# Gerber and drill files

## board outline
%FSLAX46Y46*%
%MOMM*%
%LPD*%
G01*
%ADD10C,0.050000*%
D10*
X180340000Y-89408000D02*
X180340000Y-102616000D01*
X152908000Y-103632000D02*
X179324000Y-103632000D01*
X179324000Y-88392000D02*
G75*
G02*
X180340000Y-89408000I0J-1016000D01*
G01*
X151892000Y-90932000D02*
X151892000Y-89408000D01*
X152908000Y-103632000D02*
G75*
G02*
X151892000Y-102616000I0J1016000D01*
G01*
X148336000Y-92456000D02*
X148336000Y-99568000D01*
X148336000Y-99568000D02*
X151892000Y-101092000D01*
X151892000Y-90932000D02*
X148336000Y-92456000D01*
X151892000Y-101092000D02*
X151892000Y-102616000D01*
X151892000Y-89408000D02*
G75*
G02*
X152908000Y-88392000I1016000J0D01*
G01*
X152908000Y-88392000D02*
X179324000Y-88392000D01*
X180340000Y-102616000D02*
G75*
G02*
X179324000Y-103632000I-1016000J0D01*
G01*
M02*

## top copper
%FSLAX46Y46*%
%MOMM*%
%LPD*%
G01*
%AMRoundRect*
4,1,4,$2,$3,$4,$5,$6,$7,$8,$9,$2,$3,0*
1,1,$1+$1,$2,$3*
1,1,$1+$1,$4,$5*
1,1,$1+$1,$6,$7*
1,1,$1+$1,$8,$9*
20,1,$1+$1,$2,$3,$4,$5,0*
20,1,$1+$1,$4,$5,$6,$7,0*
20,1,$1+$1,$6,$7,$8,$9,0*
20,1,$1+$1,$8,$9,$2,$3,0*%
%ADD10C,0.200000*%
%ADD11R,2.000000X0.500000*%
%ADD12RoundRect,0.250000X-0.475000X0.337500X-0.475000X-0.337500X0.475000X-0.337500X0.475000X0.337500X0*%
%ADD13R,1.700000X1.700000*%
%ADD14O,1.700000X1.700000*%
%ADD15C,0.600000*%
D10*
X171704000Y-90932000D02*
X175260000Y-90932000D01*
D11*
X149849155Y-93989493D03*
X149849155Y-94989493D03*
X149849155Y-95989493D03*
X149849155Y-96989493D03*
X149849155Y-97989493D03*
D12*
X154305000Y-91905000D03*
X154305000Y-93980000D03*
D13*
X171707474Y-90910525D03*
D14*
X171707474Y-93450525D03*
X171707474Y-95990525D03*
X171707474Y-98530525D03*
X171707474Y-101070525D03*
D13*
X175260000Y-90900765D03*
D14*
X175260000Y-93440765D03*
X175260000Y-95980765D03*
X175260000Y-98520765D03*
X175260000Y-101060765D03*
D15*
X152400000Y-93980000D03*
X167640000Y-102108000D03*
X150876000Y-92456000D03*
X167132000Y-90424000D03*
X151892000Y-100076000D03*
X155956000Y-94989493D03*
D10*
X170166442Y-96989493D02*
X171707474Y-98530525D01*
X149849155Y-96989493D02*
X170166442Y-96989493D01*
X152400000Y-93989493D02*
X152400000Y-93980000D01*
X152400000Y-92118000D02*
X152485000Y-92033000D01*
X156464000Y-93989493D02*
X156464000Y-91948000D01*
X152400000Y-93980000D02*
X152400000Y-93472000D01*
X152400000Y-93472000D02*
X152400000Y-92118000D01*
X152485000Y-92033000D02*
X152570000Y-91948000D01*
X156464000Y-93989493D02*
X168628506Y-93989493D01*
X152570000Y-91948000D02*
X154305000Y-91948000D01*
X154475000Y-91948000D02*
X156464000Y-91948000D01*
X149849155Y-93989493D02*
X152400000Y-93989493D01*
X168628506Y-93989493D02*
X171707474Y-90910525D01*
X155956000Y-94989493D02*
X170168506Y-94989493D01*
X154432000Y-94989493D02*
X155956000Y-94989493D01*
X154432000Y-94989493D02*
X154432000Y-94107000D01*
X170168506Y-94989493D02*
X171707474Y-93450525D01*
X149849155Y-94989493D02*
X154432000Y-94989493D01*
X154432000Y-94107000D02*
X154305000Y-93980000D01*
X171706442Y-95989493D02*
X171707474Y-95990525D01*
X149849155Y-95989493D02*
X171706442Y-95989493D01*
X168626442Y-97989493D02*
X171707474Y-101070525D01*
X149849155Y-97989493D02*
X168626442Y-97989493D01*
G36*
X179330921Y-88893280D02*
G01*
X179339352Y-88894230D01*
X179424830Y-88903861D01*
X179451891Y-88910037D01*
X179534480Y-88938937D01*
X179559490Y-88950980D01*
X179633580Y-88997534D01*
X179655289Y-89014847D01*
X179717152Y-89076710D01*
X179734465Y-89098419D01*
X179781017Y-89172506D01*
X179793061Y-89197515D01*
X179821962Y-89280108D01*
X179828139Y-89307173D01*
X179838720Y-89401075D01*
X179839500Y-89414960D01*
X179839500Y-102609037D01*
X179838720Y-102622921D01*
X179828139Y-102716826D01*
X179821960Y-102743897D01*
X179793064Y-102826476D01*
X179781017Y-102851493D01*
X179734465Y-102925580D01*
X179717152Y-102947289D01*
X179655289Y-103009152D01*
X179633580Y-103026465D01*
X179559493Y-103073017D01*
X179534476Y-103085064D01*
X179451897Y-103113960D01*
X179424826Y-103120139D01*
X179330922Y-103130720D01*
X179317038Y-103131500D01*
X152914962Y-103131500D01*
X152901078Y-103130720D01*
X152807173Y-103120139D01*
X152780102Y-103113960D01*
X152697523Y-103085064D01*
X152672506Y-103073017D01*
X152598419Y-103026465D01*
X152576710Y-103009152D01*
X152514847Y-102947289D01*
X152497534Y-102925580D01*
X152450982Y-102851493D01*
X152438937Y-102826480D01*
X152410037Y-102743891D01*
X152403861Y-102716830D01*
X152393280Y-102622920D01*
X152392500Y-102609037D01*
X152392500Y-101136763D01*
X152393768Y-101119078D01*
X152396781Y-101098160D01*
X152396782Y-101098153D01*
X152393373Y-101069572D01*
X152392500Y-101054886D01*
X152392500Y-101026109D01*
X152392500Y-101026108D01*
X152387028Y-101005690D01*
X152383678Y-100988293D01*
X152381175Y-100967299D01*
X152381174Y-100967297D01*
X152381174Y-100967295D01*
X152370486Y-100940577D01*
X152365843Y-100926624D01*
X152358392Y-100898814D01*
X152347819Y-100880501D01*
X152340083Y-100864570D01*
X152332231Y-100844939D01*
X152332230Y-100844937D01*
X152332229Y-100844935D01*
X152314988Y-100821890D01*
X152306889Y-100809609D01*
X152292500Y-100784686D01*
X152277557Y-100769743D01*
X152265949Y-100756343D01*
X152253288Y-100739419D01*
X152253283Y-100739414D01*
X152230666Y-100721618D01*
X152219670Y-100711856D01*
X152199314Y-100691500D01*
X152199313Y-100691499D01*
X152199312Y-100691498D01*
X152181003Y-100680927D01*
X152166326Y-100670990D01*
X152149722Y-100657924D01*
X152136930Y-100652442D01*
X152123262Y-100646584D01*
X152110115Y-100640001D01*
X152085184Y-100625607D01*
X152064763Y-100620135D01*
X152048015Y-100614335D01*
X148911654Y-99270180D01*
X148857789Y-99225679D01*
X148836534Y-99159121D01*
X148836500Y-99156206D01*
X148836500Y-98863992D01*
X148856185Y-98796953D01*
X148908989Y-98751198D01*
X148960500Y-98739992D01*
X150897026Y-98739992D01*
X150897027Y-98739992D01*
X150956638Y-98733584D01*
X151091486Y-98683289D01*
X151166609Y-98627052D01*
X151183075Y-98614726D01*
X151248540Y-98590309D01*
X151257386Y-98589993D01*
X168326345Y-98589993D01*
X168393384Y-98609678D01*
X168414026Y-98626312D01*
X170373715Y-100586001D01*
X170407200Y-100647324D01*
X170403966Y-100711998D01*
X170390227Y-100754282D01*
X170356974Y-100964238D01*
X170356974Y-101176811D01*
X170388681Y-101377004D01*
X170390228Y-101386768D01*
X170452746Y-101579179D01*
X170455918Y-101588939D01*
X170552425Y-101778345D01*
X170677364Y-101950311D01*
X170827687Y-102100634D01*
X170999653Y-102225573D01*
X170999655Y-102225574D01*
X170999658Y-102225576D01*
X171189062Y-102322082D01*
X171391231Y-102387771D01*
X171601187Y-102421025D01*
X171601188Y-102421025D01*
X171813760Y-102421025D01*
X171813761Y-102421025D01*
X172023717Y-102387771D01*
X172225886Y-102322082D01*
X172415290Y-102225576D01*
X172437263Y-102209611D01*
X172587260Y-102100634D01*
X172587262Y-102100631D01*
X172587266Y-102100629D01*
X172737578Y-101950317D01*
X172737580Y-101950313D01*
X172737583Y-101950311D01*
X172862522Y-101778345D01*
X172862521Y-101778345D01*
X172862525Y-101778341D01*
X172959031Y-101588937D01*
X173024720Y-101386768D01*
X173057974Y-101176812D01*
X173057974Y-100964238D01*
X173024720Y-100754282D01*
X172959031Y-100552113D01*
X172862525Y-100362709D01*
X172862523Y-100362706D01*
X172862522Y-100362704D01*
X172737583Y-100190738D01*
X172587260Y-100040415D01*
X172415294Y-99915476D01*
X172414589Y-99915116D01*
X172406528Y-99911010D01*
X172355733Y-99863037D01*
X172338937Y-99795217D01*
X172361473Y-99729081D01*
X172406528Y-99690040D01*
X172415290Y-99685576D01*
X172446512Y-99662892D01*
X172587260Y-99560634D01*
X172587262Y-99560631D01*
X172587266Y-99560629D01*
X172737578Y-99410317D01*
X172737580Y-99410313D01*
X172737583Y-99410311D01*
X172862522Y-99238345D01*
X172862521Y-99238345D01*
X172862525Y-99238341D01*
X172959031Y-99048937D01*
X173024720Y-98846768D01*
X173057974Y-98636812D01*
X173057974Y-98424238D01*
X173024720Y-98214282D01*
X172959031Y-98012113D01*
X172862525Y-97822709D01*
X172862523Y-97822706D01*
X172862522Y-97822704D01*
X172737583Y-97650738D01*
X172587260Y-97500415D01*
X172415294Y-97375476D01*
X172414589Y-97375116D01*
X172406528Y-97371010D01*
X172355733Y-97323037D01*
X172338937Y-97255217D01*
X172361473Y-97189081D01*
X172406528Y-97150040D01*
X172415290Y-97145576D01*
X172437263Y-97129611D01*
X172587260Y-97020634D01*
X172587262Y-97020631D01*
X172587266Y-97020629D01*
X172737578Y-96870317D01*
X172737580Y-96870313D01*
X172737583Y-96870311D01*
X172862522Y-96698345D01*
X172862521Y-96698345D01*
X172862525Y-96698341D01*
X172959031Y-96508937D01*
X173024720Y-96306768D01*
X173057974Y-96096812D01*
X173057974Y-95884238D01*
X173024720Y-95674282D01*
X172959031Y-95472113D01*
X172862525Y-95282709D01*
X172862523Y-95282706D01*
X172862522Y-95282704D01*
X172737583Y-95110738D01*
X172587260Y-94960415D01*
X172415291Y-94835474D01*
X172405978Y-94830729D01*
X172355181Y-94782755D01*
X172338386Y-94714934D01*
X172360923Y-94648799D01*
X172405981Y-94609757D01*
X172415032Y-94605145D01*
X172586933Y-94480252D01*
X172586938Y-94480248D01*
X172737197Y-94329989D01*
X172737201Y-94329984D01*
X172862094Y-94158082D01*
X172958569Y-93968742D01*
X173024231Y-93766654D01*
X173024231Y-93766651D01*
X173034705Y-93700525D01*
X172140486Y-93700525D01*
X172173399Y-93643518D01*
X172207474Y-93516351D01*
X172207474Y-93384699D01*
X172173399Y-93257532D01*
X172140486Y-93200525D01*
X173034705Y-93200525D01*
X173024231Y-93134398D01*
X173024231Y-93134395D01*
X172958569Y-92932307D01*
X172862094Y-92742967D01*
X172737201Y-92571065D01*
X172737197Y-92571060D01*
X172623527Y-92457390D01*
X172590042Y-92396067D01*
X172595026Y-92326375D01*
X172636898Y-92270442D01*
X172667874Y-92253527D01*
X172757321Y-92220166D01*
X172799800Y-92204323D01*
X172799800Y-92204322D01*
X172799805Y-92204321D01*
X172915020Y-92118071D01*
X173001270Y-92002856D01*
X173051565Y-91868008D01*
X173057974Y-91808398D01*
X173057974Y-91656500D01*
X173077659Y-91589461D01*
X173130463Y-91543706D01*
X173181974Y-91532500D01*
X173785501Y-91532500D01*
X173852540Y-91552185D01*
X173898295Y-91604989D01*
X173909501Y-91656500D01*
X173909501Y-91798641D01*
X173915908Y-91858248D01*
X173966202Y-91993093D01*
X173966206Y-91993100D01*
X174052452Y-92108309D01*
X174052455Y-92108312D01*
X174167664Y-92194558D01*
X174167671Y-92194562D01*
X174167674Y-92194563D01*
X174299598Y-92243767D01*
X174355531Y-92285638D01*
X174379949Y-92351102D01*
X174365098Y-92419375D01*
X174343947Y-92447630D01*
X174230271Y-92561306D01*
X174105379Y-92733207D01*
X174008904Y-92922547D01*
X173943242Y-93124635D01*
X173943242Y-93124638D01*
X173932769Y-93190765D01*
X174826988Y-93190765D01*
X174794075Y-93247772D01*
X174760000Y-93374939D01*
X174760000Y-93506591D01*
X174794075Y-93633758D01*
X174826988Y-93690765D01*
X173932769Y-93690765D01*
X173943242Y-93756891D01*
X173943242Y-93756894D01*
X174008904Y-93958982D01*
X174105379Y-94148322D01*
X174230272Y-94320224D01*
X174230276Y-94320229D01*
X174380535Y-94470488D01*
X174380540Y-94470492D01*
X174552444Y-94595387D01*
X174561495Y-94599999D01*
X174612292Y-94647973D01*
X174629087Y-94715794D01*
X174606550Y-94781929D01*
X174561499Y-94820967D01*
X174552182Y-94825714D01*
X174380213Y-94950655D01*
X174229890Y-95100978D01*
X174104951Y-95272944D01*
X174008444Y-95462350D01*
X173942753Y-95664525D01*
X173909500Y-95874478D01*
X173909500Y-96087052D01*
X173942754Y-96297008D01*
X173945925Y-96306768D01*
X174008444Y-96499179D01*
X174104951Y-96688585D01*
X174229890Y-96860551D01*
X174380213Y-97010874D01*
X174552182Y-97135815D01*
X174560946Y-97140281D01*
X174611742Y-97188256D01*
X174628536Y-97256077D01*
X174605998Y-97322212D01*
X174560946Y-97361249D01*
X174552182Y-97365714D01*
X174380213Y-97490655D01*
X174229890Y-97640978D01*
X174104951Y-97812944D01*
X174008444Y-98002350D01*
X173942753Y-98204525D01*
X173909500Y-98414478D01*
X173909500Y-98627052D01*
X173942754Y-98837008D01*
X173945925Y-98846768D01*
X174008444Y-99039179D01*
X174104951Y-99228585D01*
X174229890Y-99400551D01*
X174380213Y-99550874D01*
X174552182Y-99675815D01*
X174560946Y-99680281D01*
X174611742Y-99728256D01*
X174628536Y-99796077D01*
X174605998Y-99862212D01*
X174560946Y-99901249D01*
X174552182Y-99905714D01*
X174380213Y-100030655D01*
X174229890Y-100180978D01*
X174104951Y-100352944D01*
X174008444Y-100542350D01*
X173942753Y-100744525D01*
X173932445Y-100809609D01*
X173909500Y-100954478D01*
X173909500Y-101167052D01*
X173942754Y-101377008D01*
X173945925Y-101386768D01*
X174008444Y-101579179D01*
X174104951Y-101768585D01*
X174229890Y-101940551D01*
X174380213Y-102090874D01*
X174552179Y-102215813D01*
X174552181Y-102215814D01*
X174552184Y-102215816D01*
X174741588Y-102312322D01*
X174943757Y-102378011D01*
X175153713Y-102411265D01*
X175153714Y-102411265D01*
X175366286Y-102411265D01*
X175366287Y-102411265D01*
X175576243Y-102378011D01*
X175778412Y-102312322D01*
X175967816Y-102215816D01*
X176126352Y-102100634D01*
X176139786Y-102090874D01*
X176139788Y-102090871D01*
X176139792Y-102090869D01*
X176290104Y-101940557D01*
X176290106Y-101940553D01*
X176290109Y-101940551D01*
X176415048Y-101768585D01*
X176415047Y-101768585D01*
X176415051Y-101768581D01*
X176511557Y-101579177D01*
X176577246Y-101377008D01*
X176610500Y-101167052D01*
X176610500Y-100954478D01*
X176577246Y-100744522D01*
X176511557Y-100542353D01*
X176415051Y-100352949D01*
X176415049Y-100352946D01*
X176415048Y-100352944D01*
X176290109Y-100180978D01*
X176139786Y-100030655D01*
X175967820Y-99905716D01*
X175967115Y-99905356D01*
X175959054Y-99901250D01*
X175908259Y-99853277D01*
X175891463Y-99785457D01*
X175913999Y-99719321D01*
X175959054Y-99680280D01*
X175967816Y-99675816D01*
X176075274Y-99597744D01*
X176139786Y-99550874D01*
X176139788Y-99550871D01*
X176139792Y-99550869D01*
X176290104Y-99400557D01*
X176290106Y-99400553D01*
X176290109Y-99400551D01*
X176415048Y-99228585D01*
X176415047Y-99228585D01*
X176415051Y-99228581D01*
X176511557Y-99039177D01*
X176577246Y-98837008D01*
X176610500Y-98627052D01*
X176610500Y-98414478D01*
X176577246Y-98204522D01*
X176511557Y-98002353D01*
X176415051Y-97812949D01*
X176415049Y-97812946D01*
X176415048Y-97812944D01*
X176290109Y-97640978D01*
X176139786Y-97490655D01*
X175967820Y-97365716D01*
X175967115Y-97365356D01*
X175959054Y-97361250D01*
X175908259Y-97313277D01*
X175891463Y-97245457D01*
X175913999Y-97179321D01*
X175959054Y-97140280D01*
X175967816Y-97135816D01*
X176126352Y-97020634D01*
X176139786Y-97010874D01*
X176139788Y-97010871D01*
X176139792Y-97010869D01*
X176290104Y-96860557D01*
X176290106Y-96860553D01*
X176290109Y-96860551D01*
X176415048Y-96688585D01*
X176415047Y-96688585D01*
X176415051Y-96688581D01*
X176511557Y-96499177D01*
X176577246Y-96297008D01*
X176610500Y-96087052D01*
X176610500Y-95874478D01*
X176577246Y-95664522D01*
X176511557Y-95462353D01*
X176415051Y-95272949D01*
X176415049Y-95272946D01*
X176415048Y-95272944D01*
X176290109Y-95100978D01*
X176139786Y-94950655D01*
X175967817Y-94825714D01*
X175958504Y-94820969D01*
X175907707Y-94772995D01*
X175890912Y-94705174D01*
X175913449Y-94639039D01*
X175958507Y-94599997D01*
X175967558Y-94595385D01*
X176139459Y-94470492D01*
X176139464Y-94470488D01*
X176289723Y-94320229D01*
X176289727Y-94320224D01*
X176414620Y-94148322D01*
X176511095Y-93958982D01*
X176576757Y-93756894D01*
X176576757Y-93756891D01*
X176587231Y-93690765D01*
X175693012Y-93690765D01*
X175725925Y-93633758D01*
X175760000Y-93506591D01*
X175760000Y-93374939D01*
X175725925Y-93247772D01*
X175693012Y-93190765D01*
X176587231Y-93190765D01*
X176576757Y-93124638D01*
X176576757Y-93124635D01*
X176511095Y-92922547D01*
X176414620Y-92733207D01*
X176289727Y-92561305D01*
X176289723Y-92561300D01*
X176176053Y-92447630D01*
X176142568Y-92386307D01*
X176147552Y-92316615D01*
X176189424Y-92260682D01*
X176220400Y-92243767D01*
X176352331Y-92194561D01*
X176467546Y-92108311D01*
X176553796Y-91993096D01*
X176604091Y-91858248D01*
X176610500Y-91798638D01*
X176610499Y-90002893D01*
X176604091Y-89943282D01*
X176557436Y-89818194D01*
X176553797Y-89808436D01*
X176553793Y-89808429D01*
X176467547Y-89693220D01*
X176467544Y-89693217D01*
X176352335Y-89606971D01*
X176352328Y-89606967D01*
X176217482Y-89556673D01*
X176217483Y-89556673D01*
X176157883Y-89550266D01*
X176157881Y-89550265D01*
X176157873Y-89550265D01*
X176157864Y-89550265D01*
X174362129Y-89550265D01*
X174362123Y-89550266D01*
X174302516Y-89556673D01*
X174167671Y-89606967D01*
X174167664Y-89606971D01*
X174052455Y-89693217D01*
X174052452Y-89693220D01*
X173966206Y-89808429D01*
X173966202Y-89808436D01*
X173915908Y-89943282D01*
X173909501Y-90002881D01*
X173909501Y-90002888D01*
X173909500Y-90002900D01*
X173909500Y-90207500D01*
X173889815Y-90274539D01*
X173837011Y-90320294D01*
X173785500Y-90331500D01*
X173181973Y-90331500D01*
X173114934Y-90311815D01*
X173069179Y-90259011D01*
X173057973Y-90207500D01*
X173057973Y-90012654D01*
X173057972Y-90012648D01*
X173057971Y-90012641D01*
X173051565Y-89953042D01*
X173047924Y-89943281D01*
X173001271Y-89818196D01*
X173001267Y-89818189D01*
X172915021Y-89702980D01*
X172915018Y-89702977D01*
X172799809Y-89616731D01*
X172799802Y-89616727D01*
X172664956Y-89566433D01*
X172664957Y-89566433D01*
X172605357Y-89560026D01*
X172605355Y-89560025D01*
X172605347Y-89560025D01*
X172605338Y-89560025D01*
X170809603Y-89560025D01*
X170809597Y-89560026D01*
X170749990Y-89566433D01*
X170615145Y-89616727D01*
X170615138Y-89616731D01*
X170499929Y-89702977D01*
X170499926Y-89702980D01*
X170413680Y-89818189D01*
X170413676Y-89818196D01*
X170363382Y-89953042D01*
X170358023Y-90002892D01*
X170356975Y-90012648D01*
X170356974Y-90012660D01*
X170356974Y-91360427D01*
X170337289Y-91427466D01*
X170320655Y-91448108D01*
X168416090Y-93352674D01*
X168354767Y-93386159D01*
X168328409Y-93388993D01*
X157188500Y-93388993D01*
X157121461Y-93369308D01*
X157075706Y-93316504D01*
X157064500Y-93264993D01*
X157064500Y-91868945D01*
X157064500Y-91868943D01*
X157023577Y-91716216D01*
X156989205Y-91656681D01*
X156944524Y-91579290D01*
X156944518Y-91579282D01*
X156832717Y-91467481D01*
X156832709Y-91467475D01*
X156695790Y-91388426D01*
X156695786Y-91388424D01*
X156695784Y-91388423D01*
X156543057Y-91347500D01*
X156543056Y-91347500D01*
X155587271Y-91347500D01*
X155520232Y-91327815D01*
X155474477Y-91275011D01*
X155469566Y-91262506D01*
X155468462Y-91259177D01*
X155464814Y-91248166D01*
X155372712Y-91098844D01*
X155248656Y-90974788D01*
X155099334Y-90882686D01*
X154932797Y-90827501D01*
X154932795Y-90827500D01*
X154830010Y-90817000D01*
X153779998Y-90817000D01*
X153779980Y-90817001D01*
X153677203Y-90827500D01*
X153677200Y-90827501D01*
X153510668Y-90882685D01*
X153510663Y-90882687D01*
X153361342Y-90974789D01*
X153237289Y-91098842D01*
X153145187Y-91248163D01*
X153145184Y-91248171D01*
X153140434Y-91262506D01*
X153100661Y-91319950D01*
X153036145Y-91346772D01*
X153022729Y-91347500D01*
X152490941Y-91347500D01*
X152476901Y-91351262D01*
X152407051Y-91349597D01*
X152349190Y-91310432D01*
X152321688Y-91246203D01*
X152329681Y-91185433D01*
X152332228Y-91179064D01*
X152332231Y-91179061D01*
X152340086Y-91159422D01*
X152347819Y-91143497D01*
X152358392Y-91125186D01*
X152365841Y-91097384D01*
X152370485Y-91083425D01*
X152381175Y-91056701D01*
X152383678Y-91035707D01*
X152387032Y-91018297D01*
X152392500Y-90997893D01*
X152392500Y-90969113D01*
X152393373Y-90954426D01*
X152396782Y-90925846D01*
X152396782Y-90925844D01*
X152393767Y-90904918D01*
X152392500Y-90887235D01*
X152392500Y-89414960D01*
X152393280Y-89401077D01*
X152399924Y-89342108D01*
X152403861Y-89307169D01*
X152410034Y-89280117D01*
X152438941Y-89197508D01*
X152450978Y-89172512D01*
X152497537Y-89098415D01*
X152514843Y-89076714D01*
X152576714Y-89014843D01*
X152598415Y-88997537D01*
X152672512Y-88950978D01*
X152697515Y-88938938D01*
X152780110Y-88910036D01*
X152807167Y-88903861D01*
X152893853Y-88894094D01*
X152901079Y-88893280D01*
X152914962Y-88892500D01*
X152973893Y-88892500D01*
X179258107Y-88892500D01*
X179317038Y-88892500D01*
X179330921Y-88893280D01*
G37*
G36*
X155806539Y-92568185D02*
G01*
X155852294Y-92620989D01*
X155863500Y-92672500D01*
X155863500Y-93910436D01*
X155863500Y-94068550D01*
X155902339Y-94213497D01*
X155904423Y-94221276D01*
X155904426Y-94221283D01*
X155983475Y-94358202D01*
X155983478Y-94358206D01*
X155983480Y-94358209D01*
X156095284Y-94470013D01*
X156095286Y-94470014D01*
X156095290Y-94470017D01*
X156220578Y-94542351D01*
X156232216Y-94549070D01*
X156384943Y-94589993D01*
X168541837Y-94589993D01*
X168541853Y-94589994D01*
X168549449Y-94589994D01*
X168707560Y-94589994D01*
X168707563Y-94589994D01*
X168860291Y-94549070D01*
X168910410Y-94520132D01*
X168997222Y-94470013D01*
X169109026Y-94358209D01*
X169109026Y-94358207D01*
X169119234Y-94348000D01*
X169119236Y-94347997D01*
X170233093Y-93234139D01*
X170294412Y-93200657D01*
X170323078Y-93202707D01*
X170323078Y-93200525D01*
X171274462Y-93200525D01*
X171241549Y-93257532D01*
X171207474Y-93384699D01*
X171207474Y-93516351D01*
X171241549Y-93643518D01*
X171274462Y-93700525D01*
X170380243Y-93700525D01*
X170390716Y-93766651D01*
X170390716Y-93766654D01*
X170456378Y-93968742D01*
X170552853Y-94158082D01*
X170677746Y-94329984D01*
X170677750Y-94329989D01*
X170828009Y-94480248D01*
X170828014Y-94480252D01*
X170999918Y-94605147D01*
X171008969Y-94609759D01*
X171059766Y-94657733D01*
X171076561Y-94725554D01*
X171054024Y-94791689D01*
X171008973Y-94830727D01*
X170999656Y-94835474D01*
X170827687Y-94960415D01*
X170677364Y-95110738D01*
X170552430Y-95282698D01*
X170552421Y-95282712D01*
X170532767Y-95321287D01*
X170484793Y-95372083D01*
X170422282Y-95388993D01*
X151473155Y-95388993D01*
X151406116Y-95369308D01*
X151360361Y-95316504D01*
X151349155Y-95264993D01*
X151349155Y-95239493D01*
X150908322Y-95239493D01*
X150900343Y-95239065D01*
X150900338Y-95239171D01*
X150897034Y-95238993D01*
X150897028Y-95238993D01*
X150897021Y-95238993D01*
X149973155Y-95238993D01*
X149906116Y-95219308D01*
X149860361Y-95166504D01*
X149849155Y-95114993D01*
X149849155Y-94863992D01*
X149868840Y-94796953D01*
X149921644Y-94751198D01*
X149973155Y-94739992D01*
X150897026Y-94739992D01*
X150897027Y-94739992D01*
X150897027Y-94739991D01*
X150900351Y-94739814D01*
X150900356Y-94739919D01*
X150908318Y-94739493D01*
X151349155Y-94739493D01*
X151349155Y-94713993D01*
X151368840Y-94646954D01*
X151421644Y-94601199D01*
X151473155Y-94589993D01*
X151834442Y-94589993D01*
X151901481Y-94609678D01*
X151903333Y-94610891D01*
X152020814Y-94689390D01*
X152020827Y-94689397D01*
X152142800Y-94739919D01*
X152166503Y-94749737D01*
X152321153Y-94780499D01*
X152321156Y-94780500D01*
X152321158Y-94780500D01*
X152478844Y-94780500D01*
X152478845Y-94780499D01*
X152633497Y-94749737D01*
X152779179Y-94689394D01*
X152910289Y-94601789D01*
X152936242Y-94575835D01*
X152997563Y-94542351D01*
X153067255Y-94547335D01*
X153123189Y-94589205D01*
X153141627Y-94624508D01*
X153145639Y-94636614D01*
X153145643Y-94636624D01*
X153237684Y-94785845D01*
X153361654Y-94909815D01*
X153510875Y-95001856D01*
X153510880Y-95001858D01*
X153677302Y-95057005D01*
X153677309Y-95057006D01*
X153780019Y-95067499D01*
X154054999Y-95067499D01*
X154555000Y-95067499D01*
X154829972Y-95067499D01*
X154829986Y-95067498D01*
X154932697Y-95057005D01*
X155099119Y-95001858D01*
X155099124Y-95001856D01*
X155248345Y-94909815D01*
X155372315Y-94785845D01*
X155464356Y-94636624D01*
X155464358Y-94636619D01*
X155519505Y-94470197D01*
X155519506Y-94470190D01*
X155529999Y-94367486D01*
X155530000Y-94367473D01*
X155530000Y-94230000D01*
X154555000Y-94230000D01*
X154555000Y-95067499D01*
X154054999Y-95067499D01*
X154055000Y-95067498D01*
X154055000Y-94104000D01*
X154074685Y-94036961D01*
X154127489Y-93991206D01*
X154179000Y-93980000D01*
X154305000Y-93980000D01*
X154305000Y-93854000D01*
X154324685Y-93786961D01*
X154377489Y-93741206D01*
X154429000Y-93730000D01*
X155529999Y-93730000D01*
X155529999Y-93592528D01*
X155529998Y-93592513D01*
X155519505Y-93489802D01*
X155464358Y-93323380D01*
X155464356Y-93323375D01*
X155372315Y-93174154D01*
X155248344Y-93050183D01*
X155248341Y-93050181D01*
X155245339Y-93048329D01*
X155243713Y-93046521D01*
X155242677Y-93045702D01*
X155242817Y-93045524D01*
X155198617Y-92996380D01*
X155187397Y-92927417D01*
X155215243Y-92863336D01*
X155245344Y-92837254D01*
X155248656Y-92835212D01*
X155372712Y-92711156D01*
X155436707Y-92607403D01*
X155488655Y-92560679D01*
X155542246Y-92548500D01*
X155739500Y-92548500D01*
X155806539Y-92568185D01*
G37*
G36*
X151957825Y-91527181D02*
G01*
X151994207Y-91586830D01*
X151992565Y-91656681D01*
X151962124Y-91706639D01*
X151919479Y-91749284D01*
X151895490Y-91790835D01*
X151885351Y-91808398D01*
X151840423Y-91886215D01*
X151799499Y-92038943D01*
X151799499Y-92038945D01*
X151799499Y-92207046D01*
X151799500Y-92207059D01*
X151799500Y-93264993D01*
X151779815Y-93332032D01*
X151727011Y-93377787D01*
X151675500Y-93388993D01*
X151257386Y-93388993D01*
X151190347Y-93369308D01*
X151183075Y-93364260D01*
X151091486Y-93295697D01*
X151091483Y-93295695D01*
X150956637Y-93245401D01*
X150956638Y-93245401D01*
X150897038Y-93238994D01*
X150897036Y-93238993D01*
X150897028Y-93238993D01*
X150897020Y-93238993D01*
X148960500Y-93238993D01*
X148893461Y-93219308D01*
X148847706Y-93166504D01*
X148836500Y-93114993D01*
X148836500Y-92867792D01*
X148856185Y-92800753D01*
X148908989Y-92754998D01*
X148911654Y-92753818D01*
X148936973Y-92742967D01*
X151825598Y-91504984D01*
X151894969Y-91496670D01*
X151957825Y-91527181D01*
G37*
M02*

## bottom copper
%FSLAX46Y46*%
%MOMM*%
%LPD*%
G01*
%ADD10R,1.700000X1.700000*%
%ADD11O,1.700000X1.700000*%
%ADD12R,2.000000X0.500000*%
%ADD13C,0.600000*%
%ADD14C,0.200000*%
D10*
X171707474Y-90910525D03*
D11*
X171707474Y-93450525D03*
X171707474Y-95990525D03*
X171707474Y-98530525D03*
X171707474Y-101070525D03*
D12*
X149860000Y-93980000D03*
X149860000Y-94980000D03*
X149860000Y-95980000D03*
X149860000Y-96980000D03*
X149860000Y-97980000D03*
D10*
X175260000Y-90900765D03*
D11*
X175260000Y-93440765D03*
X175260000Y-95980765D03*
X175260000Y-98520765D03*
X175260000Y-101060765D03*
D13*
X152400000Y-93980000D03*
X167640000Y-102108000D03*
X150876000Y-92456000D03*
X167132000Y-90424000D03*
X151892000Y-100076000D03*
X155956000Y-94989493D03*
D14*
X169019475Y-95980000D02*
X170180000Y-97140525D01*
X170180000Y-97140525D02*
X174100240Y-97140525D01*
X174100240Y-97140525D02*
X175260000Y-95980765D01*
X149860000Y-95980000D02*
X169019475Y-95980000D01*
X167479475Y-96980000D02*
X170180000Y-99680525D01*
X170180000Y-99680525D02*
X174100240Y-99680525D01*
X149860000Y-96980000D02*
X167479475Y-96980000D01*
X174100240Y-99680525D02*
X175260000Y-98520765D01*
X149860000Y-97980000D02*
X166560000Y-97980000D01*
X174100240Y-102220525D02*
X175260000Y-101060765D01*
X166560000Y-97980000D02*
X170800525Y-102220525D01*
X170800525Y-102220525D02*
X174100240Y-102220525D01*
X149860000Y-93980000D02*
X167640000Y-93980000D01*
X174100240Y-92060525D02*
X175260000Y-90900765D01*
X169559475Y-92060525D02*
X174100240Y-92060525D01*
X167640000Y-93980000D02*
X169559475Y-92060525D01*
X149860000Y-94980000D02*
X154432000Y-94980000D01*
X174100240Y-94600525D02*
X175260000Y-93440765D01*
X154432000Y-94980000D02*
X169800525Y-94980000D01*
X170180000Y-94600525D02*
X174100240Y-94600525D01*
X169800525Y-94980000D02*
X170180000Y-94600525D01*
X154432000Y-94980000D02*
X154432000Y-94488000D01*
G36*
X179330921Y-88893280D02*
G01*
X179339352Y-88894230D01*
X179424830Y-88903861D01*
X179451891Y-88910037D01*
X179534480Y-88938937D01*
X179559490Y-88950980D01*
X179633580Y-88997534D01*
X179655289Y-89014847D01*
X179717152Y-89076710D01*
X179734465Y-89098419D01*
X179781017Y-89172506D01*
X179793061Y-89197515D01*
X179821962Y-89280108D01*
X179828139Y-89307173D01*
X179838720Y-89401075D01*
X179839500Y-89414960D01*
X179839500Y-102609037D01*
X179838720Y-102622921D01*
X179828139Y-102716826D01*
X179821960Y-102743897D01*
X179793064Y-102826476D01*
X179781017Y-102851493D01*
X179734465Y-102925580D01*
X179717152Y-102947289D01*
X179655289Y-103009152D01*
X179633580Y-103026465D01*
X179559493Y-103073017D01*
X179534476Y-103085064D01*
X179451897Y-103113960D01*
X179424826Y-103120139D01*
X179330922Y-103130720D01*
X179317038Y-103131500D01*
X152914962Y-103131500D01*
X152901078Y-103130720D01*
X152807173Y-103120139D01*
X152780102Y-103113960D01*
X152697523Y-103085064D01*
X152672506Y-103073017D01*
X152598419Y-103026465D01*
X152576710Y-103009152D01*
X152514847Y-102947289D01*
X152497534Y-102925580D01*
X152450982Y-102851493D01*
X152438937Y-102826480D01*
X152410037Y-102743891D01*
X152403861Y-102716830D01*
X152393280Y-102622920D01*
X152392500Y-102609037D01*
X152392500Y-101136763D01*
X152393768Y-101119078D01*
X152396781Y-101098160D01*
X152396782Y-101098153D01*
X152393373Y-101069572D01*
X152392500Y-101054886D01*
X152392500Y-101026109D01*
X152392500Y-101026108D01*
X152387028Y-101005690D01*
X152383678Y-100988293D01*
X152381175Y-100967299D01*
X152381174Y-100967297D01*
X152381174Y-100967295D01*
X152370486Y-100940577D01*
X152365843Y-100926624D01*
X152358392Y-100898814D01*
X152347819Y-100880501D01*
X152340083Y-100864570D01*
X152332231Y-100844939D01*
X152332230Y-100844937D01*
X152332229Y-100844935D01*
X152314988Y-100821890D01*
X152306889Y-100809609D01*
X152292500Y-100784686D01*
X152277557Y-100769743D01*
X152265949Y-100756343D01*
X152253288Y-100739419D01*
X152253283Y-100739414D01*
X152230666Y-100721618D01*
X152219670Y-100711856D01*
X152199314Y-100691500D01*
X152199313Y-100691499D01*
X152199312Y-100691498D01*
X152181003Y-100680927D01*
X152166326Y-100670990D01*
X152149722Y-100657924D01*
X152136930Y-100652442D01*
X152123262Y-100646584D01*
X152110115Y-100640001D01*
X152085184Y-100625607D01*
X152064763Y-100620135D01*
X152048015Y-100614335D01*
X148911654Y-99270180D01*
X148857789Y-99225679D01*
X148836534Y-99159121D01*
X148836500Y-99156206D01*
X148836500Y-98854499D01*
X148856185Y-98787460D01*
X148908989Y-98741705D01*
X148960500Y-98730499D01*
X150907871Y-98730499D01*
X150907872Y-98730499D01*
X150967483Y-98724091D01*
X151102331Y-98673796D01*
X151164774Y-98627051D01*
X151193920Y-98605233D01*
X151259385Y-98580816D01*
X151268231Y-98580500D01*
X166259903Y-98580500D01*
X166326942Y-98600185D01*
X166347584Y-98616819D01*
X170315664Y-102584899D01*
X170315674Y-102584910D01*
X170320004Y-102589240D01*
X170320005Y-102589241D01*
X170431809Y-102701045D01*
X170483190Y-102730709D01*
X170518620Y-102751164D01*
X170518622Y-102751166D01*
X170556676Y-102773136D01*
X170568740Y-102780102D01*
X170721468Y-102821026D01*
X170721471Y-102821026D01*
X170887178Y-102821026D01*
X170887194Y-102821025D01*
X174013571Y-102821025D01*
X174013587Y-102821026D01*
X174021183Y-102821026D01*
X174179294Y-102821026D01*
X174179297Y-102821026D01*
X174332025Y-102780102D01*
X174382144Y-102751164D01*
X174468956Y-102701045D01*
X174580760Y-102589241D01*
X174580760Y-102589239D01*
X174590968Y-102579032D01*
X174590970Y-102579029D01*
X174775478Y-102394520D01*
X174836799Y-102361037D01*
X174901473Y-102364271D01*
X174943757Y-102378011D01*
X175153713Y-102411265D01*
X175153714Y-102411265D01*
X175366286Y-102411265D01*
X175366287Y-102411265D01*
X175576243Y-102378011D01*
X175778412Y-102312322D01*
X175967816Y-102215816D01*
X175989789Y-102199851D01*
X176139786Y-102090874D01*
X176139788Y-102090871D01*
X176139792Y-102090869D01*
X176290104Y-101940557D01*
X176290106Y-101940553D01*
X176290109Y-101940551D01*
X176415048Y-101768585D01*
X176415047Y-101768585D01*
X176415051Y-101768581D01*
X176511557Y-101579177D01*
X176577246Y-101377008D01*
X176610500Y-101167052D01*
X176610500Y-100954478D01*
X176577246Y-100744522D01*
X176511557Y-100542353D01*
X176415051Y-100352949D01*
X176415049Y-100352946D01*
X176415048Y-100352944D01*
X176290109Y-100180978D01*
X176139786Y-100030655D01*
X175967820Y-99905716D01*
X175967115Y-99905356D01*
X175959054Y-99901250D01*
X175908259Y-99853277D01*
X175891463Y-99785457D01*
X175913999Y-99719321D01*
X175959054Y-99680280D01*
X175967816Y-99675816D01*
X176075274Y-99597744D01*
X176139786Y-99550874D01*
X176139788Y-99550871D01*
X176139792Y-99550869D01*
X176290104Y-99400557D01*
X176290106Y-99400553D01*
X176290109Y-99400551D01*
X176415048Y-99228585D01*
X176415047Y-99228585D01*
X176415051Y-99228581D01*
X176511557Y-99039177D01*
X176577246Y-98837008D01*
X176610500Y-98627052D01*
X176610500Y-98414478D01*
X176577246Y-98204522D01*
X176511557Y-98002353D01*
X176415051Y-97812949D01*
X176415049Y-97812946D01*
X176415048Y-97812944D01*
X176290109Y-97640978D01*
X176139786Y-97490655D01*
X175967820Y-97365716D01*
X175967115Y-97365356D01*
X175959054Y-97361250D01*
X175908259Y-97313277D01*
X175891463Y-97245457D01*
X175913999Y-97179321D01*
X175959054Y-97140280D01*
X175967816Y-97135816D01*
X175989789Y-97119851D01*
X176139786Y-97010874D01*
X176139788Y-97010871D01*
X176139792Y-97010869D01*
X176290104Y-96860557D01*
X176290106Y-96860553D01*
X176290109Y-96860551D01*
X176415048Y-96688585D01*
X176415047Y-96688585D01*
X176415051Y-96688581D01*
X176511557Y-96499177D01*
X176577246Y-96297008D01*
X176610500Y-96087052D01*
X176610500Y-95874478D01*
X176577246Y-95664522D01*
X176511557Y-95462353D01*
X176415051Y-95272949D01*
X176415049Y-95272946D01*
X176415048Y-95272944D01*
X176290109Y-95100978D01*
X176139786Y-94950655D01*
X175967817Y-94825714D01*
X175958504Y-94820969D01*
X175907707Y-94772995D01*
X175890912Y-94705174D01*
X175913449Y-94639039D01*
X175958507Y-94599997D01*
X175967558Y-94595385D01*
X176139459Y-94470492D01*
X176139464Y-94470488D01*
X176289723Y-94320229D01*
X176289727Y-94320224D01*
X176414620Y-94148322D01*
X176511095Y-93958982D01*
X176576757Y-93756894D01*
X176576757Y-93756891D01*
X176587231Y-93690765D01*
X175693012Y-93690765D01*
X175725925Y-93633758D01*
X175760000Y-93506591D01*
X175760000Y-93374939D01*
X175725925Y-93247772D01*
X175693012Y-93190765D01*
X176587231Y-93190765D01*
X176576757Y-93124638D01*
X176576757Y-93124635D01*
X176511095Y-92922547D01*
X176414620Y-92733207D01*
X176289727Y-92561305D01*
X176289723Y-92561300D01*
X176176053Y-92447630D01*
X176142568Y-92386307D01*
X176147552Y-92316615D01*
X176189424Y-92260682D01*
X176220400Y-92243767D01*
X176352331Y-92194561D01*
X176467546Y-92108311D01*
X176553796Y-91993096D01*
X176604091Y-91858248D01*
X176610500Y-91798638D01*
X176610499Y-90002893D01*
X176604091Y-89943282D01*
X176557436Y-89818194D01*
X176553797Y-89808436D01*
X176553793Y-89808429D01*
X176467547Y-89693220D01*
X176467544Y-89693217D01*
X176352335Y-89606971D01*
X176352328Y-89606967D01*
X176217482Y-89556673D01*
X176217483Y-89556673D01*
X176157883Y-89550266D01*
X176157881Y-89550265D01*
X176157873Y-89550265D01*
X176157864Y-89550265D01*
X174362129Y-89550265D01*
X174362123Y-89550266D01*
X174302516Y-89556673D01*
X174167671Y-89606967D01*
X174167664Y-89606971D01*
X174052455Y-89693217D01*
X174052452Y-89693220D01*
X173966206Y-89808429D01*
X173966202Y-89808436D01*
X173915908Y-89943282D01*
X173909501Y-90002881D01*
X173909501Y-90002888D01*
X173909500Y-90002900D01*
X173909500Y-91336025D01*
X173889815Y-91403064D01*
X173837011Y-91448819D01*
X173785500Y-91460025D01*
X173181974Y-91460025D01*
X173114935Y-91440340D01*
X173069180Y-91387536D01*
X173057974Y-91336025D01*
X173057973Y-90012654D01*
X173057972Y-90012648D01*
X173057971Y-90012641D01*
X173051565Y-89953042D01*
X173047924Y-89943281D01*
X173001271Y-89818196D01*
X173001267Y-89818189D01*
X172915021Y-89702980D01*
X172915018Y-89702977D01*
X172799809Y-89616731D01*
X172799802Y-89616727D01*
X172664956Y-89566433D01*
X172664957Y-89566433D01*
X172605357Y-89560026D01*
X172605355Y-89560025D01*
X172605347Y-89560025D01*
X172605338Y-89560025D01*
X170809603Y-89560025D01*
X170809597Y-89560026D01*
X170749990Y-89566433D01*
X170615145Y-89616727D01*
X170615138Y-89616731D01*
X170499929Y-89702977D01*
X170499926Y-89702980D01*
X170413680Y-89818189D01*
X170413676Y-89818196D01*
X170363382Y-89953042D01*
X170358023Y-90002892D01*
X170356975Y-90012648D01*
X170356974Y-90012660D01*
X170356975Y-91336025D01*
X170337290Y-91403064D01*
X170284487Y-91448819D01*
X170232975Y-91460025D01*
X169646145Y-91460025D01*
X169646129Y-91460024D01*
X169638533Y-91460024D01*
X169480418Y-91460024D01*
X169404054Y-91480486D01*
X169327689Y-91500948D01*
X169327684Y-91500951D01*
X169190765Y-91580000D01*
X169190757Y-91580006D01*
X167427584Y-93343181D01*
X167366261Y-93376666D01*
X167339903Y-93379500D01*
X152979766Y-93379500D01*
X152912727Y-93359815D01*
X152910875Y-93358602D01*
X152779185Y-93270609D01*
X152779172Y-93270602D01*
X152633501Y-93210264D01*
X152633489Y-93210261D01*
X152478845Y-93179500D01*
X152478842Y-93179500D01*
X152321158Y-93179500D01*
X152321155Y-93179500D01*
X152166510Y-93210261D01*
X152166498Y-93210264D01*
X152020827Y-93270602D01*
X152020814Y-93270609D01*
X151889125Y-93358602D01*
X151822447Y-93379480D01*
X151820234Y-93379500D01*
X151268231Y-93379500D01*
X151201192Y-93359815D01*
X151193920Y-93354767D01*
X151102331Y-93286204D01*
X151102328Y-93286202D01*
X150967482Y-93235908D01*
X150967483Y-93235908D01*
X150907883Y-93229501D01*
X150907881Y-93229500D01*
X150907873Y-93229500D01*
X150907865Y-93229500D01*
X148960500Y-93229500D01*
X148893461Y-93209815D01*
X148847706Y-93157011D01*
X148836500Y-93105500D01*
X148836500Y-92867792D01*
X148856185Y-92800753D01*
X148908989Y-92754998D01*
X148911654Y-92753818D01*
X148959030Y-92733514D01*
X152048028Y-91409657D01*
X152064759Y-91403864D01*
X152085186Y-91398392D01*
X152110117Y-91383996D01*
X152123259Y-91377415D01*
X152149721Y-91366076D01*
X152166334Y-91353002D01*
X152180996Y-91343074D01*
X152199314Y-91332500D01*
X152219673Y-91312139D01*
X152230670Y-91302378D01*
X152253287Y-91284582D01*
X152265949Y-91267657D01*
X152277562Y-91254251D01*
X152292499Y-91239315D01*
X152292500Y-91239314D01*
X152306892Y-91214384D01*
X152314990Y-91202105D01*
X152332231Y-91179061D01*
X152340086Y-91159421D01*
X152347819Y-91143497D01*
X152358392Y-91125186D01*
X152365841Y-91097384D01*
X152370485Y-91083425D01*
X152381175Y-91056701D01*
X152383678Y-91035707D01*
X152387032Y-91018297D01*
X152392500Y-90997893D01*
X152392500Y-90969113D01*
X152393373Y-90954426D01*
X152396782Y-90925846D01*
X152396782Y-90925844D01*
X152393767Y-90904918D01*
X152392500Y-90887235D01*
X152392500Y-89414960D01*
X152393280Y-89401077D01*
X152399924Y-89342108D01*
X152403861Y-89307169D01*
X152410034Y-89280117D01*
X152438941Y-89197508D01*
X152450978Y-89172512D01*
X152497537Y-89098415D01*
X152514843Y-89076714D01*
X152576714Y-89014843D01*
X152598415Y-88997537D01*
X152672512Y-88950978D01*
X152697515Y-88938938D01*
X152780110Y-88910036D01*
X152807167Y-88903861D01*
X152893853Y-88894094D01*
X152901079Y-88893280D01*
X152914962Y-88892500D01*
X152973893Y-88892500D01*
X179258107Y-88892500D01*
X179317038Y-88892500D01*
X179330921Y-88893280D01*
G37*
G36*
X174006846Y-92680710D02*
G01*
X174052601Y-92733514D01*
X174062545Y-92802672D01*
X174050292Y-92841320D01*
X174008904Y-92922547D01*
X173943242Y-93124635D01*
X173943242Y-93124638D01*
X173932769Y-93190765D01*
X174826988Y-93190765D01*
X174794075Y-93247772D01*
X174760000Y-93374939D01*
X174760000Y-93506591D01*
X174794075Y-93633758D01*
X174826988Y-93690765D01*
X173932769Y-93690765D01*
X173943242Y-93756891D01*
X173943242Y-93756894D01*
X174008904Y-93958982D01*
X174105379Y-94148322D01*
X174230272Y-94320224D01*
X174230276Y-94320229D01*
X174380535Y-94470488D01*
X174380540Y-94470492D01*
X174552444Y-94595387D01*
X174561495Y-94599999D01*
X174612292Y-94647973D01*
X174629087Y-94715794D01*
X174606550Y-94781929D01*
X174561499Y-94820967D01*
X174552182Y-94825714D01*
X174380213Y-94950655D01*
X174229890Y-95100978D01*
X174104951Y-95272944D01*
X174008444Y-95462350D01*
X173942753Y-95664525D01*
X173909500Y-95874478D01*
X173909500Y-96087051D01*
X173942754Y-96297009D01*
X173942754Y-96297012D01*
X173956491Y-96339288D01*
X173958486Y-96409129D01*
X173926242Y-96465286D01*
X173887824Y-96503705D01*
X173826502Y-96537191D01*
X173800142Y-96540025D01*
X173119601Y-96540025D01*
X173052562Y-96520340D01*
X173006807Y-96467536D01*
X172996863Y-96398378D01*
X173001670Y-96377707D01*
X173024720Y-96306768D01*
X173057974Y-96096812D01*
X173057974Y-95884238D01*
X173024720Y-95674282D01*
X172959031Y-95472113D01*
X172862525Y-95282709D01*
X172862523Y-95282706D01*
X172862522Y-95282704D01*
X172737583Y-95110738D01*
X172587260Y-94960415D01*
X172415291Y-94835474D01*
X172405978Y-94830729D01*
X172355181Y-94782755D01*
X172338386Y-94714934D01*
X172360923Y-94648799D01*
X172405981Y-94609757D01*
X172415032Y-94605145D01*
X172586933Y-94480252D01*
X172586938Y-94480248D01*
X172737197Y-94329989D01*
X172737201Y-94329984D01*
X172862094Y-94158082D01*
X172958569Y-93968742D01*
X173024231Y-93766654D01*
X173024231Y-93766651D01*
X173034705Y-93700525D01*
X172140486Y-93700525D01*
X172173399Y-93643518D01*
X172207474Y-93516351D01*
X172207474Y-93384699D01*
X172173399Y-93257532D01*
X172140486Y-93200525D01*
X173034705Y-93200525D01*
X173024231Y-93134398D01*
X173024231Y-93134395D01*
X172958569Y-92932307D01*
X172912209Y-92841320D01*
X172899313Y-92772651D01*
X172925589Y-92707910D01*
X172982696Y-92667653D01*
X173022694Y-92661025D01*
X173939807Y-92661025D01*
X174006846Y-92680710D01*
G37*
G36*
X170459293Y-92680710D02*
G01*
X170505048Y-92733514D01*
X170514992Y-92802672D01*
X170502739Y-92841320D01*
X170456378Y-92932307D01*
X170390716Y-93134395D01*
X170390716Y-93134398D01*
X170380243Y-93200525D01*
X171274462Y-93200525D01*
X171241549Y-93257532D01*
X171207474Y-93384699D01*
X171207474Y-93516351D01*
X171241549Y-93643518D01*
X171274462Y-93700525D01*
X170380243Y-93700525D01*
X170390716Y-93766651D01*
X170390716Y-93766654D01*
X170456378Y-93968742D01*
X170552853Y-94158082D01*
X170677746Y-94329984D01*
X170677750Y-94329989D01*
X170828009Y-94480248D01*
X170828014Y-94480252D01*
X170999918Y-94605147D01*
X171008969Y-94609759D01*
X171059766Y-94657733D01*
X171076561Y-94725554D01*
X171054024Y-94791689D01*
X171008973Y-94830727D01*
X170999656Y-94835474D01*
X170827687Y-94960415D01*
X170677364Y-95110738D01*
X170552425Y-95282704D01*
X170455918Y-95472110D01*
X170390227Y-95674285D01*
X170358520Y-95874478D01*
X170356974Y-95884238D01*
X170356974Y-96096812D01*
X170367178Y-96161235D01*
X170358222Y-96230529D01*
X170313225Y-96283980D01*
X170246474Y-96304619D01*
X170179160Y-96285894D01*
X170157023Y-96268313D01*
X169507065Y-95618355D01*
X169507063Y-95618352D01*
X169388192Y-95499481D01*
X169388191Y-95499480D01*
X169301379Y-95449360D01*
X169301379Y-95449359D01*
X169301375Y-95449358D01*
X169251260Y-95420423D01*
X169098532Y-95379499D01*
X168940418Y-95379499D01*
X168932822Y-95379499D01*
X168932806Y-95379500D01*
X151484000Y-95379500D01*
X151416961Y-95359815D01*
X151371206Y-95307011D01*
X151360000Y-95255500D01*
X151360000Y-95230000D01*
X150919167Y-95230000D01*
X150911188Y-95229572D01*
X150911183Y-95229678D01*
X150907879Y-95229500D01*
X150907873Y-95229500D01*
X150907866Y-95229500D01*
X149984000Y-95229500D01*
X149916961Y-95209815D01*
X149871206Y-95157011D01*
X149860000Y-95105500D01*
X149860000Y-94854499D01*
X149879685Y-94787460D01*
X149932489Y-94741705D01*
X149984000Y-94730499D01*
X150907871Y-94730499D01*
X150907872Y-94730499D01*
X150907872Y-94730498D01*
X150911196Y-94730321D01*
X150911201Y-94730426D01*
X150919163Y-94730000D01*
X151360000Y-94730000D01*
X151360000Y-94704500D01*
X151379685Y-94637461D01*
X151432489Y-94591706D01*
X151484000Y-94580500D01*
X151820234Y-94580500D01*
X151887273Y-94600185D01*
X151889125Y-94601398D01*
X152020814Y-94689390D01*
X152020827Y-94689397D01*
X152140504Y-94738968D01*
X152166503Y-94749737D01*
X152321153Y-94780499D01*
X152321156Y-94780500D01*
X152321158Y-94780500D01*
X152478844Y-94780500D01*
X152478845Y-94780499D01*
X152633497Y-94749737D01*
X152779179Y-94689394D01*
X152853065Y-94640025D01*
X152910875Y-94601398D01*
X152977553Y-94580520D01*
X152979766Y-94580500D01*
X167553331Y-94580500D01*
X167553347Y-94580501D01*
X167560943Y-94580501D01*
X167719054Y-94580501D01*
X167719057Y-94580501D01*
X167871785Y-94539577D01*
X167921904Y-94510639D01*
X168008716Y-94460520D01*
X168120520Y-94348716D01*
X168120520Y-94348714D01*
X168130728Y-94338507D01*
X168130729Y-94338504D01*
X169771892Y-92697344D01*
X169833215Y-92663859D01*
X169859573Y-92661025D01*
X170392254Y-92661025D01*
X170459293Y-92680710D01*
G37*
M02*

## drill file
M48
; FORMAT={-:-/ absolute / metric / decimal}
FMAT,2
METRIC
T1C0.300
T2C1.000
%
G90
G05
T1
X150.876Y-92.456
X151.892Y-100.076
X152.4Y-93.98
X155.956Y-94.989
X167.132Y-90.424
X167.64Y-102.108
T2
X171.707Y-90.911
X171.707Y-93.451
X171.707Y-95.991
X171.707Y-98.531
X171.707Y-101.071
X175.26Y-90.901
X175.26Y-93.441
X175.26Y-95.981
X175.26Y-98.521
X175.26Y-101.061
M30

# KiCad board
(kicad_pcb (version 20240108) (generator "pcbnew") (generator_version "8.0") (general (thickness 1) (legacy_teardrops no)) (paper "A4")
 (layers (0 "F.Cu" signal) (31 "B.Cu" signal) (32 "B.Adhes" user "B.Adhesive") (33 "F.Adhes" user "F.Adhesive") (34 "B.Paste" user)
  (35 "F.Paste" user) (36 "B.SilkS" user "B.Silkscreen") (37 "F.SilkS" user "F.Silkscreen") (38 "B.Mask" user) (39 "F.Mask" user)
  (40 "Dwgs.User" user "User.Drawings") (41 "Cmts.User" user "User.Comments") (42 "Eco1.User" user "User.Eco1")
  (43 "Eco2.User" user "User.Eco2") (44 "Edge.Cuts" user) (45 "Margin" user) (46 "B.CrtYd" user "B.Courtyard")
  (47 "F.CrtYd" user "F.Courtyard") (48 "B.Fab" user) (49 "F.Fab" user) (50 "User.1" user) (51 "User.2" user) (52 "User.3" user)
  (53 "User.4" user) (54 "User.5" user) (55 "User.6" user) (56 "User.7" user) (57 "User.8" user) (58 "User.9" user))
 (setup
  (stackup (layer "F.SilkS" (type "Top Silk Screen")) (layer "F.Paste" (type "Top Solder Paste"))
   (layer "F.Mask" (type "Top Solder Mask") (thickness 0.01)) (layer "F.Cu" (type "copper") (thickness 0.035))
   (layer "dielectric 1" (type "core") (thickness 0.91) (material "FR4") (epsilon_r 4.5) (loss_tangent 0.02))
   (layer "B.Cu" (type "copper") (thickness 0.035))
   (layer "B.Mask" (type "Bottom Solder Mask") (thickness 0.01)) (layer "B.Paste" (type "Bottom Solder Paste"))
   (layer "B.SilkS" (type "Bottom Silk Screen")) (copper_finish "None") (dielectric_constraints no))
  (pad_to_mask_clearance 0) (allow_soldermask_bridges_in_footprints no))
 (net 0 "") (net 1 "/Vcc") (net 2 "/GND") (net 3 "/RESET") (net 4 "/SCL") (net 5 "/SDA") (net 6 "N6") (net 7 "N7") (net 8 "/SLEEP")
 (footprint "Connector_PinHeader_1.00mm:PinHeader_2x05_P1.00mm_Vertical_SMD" (layer "F.Cu") (at 149.874555 95.941493)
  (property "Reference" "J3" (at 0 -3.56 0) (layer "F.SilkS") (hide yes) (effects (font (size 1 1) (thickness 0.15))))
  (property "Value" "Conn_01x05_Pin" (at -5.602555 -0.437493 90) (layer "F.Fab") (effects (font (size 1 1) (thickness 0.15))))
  (pad "1" smd rect (at -0.0254 -1.952) (size 2 0.5) (layers "F.Cu" "F.Paste" "F.Mask") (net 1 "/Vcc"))
  (pad "2" smd rect (at -0.0254 -0.952) (size 2 0.5) (layers "F.Cu" "F.Paste" "F.Mask") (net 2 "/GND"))
  (pad "3" smd rect (at -0.0254 0.048) (size 2 0.5) (layers "F.Cu" "F.Paste" "F.Mask") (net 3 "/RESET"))
  (pad "4" smd rect (at -0.0254 1.048) (size 2 0.5) (layers "F.Cu" "F.Paste" "F.Mask") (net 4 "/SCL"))
  (pad "5" smd rect (at -0.0254 2.048) (size 2 0.5) (layers "F.Cu" "F.Paste" "F.Mask") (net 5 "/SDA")))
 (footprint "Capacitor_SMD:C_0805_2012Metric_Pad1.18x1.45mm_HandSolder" (layer "F.Cu") (at 154.305 92.9425 -90)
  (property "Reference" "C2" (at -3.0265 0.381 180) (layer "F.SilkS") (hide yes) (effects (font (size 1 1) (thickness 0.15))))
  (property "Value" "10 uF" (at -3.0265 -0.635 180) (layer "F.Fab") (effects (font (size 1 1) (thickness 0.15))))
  (pad "1" smd roundrect (at -1.0375 0 270) (size 1.175 1.45) (layers "F.Cu" "F.Paste" "F.Mask") (roundrect_rratio 0.212766) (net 1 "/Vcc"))
  (pad "2" smd roundrect (at 1.0375 0 270) (size 1.175 1.45) (layers "F.Cu" "F.Paste" "F.Mask") (roundrect_rratio 0.212766) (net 2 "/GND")))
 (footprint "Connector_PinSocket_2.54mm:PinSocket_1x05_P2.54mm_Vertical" (layer "F.Cu") (at 171.707474 90.910525)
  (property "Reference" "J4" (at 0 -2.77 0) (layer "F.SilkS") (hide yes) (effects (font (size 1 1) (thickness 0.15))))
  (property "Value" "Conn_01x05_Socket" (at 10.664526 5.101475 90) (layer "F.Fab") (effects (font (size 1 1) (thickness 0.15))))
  (pad "1" thru_hole rect (at 0 0) (size 1.7 1.7) (drill 1) (layers "*.Cu" "*.Mask") (remove_unused_layers no) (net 1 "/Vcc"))
  (pad "2" thru_hole oval (at 0 2.54) (size 1.7 1.7) (drill 1) (layers "*.Cu" "*.Mask") (remove_unused_layers no) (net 2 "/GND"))
  (pad "3" thru_hole oval (at 0 5.08) (size 1.7 1.7) (drill 1) (layers "*.Cu" "*.Mask") (remove_unused_layers no) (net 3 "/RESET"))
  (pad "4" thru_hole oval (at 0 7.62) (size 1.7 1.7) (drill 1) (layers "*.Cu" "*.Mask") (remove_unused_layers no) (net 4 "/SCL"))
  (pad "5" thru_hole oval (at 0 10.16) (size 1.7 1.7) (drill 1) (layers "*.Cu" "*.Mask") (remove_unused_layers no) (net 5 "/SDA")))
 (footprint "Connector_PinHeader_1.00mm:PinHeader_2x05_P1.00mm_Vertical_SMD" (layer "B.Cu") (at 149.86 96.0054 180)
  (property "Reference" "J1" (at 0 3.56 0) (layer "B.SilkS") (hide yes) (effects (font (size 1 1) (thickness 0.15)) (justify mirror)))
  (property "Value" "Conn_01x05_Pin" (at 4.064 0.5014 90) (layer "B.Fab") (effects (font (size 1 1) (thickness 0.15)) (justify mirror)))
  (pad "1" smd rect (at 0 2.0254 180) (size 2 0.5) (layers "B.Cu" "B.Paste" "B.Mask") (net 1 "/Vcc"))
  (pad "2" smd rect (at 0 1.0254 180) (size 2 0.5) (layers "B.Cu" "B.Paste" "B.Mask") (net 2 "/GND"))
  (pad "3" smd rect (at 0 0.0254 180) (size 2 0.5) (layers "B.Cu" "B.Paste" "B.Mask") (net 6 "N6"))
  (pad "4" smd rect (at 0 -0.9746 180) (size 2 0.5) (layers "B.Cu" "B.Paste" "B.Mask") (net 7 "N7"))
  (pad "5" smd rect (at 0 -1.9746 180) (size 2 0.5) (layers "B.Cu" "B.Paste" "B.Mask") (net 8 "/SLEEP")))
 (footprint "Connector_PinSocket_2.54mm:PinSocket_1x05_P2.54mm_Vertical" (layer "B.Cu") (at 175.26 90.900765 180)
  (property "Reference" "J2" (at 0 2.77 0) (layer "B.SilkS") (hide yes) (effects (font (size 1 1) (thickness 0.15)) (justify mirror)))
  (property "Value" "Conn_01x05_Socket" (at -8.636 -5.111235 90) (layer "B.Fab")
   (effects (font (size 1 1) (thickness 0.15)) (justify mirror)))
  (pad "1" thru_hole rect (at 0 0 180) (size 1.7 1.7) (drill 1) (layers "*.Cu" "*.Mask") (remove_unused_layers no) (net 1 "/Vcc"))
  (pad "2" thru_hole oval (at 0 -2.54 180) (size 1.7 1.7) (drill 1) (layers "*.Cu" "*.Mask") (remove_unused_layers no) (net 2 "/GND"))
  (pad "3" thru_hole oval (at 0 -5.08 180) (size 1.7 1.7) (drill 1) (layers "*.Cu" "*.Mask") (remove_unused_layers no) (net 6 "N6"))
  (pad "4" thru_hole oval (at 0 -7.62 180) (size 1.7 1.7) (drill 1) (layers "*.Cu" "*.Mask") (remove_unused_layers no) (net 7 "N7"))
  (pad "5" thru_hole oval (at 0 -10.16 180) (size 1.7 1.7) (drill 1) (layers "*.Cu" "*.Mask") (remove_unused_layers no) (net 8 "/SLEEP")))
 (gr_line (start 171.704 90.932) (end 175.26 90.932) (stroke (width 0.2) (type default)) (layer "F.Cu") (net 1))
 (gr_line (start 180.34 89.408) (end 180.34 102.616) (stroke (width 0.05) (type default)) (layer "Edge.Cuts"))
 (gr_line (start 152.908 103.632) (end 179.324 103.632) (stroke (width 0.05) (type default)) (layer "Edge.Cuts"))
 (gr_arc (start 179.324 88.392) (mid 180.04242 88.68958) (end 180.34 89.408) (stroke (width 0.05) (type default)) (layer "Edge.Cuts"))
 (gr_line (start 151.892 90.932) (end 151.892 89.408) (stroke (width 0.05) (type default)) (layer "Edge.Cuts"))
 (gr_arc (start 152.908 103.632) (mid 152.18958 103.33442) (end 151.892 102.616) (stroke (width 0.05) (type default)) (layer "Edge.Cuts"))
 (gr_line (start 148.336 92.456) (end 148.336 99.568) (stroke (width 0.05) (type default)) (layer "Edge.Cuts"))
 (gr_line (start 148.336 99.568) (end 151.892 101.092) (stroke (width 0.05) (type default)) (layer "Edge.Cuts"))
 (gr_line (start 151.892 90.932) (end 148.336 92.456) (stroke (width 0.05) (type default)) (layer "Edge.Cuts"))
 (gr_line (start 151.892 101.092) (end 151.892 102.616) (stroke (width 0.05) (type default)) (layer "Edge.Cuts"))
 (gr_arc (start 151.892 89.408) (mid 152.18958 88.68958) (end 152.908 88.392) (stroke (width 0.05) (type default)) (layer "Edge.Cuts"))
 (gr_line (start 152.908 88.392) (end 179.324 88.392) (stroke (width 0.05) (type default)) (layer "Edge.Cuts"))
 (gr_arc (start 180.34 102.616) (mid 180.04242 103.33442) (end 179.324 103.632) (stroke (width 0.05) (type default)) (layer "Edge.Cuts"))
 (segment (start 169.019475 95.98) (end 170.18 97.140525) (width 0.2) (layer "B.Cu") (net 6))
 (segment (start 170.18 97.140525) (end 174.10024 97.140525) (width 0.2) (layer "B.Cu") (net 6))
 (segment (start 174.10024 97.140525) (end 175.26 95.980765) (width 0.2) (layer "B.Cu") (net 6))
 (segment (start 149.86 95.98) (end 169.019475 95.98) (width 0.2) (layer "B.Cu") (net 6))
 (segment (start 167.479475 96.98) (end 170.18 99.680525) (width 0.2) (layer "B.Cu") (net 7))
 (segment (start 170.18 99.680525) (end 174.10024 99.680525) (width 0.2) (layer "B.Cu") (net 7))
 (segment (start 149.86 96.98) (end 167.479475 96.98) (width 0.2) (layer "B.Cu") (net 7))
 (segment (start 174.10024 99.680525) (end 175.26 98.520765) (width 0.2) (layer "B.Cu") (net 7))
 (segment (start 149.86 97.98) (end 166.56 97.98) (width 0.2) (layer "B.Cu") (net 8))
 (segment (start 174.10024 102.220525) (end 175.26 101.060765) (width 0.2) (layer "B.Cu") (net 8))
 (segment (start 166.56 97.98) (end 170.800525 102.220525) (width 0.2) (layer "B.Cu") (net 8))
 (segment (start 170.800525 102.220525) (end 174.10024 102.220525) (width 0.2) (layer "B.Cu") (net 8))
 (segment (start 170.166442 96.989493) (end 171.707474 98.530525) (width 0.2) (layer "F.Cu") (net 4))
 (segment (start 149.849155 96.989493) (end 170.166442 96.989493) (width 0.2) (layer "F.Cu") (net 4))
 (segment (start 152.4 93.989493) (end 152.4 93.98) (width 0.2) (layer "F.Cu") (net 1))
 (segment (start 152.4 92.118) (end 152.485 92.033) (width 0.2) (layer "F.Cu") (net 1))
 (segment (start 156.464 93.989493) (end 156.464 91.948) (width 0.2) (layer "F.Cu") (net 1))
 (segment (start 152.4 93.98) (end 152.4 93.472) (width 0.2) (layer "F.Cu") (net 1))
 (segment (start 152.4 93.472) (end 152.4 92.118) (width 0.2) (layer "F.Cu") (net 1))
 (segment (start 152.485 92.033) (end 152.57 91.948) (width 0.2) (layer "F.Cu") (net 1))
 (segment (start 156.464 93.989493) (end 168.628506 93.989493) (width 0.2) (layer "F.Cu") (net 1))
 (segment (start 152.57 91.948) (end 154.305 91.948) (width 0.2) (layer "F.Cu") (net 1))
 (segment (start 154.475 91.948) (end 156.464 91.948) (width 0.2) (layer "F.Cu") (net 1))
 (segment (start 149.849155 93.989493) (end 152.4 93.989493) (width 0.2) (layer "F.Cu") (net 1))
 (segment (start 168.628506 93.989493) (end 171.707474 90.910525) (width 0.2) (layer "F.Cu") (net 1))
 (via (at 152.4 93.98) (size 0.6) (drill 0.3) (layers "F.Cu" "B.Cu") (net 1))
 (segment (start 149.86 93.98) (end 167.64 93.98) (width 0.2) (layer "B.Cu") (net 1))
 (segment (start 174.10024 92.060525) (end 175.26 90.900765) (width 0.2) (layer "B.Cu") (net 1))
 (segment (start 169.559475 92.060525) (end 174.10024 92.060525) (width 0.2) (layer "B.Cu") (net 1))
 (segment (start 167.64 93.98) (end 169.559475 92.060525) (width 0.2) (layer "B.Cu") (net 1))
 (segment (start 155.956 94.989493) (end 170.168506 94.989493) (width 0.2) (layer "F.Cu") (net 2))
 (segment (start 154.432 94.989493) (end 155.956 94.989493) (width 0.2) (layer "F.Cu") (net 2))
 (segment (start 154.432 94.989493) (end 154.432 94.107) (width 0.2) (layer "F.Cu") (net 2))
 (segment (start 170.168506 94.989493) (end 171.707474 93.450525) (width 0.2) (layer "F.Cu") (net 2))
 (segment (start 149.849155 94.989493) (end 154.432 94.989493) (width 0.2) (layer "F.Cu") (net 2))
 (segment (start 154.432 94.107) (end 154.305 93.98) (width 0.2) (layer "F.Cu") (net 2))
 (via (at 167.64 102.108) (size 0.6) (drill 0.3) (layers "F.Cu" "B.Cu") (free yes) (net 2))
 (via (at 150.876 92.456) (size 0.6) (drill 0.3) (layers "F.Cu" "B.Cu") (free yes) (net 2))
 (via (at 167.132 90.424) (size 0.6) (drill 0.3) (layers "F.Cu" "B.Cu") (free yes) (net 2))
 (via (at 151.892 100.076) (size 0.6) (drill 0.3) (layers "F.Cu" "B.Cu") (free yes) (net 2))
 (via (at 155.956 94.989493) (size 0.6) (drill 0.3) (layers "F.Cu" "B.Cu") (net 2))
 (segment (start 149.86 94.98) (end 154.432 94.98) (width 0.2) (layer "B.Cu") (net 2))
 (segment (start 174.10024 94.600525) (end 175.26 93.440765) (width 0.2) (layer "B.Cu") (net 2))
 (segment (start 154.432 94.98) (end 169.800525 94.98) (width 0.2) (layer "B.Cu") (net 2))
 (segment (start 170.18 94.600525) (end 174.10024 94.600525) (width 0.2) (layer "B.Cu") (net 2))
 (segment (start 169.800525 94.98) (end 170.18 94.600525) (width 0.2) (layer "B.Cu") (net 2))
 (segment (start 154.432 94.98) (end 154.432 94.488) (width 0.2) (layer "B.Cu") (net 2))
 (segment (start 171.706442 95.989493) (end 171.707474 95.990525) (width 0.2) (layer "F.Cu") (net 3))
 (segment (start 149.849155 95.989493) (end 171.706442 95.989493) (width 0.2) (layer "F.Cu") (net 3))
 (segment (start 168.626442 97.989493) (end 171.707474 101.070525) (width 0.2) (layer "F.Cu") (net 5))
 (segment (start 149.849155 97.989493) (end 168.626442 97.989493) (width 0.2) (layer "F.Cu") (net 5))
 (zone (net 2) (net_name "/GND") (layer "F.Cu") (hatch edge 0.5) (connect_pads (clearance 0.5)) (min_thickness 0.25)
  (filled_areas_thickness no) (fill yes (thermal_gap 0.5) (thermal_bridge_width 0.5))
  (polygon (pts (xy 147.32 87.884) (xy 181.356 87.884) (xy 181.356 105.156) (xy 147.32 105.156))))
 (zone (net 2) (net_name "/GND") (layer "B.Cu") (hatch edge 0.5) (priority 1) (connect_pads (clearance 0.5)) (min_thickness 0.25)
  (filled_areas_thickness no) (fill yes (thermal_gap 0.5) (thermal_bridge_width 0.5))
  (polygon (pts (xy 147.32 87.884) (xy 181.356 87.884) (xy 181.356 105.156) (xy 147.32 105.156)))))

